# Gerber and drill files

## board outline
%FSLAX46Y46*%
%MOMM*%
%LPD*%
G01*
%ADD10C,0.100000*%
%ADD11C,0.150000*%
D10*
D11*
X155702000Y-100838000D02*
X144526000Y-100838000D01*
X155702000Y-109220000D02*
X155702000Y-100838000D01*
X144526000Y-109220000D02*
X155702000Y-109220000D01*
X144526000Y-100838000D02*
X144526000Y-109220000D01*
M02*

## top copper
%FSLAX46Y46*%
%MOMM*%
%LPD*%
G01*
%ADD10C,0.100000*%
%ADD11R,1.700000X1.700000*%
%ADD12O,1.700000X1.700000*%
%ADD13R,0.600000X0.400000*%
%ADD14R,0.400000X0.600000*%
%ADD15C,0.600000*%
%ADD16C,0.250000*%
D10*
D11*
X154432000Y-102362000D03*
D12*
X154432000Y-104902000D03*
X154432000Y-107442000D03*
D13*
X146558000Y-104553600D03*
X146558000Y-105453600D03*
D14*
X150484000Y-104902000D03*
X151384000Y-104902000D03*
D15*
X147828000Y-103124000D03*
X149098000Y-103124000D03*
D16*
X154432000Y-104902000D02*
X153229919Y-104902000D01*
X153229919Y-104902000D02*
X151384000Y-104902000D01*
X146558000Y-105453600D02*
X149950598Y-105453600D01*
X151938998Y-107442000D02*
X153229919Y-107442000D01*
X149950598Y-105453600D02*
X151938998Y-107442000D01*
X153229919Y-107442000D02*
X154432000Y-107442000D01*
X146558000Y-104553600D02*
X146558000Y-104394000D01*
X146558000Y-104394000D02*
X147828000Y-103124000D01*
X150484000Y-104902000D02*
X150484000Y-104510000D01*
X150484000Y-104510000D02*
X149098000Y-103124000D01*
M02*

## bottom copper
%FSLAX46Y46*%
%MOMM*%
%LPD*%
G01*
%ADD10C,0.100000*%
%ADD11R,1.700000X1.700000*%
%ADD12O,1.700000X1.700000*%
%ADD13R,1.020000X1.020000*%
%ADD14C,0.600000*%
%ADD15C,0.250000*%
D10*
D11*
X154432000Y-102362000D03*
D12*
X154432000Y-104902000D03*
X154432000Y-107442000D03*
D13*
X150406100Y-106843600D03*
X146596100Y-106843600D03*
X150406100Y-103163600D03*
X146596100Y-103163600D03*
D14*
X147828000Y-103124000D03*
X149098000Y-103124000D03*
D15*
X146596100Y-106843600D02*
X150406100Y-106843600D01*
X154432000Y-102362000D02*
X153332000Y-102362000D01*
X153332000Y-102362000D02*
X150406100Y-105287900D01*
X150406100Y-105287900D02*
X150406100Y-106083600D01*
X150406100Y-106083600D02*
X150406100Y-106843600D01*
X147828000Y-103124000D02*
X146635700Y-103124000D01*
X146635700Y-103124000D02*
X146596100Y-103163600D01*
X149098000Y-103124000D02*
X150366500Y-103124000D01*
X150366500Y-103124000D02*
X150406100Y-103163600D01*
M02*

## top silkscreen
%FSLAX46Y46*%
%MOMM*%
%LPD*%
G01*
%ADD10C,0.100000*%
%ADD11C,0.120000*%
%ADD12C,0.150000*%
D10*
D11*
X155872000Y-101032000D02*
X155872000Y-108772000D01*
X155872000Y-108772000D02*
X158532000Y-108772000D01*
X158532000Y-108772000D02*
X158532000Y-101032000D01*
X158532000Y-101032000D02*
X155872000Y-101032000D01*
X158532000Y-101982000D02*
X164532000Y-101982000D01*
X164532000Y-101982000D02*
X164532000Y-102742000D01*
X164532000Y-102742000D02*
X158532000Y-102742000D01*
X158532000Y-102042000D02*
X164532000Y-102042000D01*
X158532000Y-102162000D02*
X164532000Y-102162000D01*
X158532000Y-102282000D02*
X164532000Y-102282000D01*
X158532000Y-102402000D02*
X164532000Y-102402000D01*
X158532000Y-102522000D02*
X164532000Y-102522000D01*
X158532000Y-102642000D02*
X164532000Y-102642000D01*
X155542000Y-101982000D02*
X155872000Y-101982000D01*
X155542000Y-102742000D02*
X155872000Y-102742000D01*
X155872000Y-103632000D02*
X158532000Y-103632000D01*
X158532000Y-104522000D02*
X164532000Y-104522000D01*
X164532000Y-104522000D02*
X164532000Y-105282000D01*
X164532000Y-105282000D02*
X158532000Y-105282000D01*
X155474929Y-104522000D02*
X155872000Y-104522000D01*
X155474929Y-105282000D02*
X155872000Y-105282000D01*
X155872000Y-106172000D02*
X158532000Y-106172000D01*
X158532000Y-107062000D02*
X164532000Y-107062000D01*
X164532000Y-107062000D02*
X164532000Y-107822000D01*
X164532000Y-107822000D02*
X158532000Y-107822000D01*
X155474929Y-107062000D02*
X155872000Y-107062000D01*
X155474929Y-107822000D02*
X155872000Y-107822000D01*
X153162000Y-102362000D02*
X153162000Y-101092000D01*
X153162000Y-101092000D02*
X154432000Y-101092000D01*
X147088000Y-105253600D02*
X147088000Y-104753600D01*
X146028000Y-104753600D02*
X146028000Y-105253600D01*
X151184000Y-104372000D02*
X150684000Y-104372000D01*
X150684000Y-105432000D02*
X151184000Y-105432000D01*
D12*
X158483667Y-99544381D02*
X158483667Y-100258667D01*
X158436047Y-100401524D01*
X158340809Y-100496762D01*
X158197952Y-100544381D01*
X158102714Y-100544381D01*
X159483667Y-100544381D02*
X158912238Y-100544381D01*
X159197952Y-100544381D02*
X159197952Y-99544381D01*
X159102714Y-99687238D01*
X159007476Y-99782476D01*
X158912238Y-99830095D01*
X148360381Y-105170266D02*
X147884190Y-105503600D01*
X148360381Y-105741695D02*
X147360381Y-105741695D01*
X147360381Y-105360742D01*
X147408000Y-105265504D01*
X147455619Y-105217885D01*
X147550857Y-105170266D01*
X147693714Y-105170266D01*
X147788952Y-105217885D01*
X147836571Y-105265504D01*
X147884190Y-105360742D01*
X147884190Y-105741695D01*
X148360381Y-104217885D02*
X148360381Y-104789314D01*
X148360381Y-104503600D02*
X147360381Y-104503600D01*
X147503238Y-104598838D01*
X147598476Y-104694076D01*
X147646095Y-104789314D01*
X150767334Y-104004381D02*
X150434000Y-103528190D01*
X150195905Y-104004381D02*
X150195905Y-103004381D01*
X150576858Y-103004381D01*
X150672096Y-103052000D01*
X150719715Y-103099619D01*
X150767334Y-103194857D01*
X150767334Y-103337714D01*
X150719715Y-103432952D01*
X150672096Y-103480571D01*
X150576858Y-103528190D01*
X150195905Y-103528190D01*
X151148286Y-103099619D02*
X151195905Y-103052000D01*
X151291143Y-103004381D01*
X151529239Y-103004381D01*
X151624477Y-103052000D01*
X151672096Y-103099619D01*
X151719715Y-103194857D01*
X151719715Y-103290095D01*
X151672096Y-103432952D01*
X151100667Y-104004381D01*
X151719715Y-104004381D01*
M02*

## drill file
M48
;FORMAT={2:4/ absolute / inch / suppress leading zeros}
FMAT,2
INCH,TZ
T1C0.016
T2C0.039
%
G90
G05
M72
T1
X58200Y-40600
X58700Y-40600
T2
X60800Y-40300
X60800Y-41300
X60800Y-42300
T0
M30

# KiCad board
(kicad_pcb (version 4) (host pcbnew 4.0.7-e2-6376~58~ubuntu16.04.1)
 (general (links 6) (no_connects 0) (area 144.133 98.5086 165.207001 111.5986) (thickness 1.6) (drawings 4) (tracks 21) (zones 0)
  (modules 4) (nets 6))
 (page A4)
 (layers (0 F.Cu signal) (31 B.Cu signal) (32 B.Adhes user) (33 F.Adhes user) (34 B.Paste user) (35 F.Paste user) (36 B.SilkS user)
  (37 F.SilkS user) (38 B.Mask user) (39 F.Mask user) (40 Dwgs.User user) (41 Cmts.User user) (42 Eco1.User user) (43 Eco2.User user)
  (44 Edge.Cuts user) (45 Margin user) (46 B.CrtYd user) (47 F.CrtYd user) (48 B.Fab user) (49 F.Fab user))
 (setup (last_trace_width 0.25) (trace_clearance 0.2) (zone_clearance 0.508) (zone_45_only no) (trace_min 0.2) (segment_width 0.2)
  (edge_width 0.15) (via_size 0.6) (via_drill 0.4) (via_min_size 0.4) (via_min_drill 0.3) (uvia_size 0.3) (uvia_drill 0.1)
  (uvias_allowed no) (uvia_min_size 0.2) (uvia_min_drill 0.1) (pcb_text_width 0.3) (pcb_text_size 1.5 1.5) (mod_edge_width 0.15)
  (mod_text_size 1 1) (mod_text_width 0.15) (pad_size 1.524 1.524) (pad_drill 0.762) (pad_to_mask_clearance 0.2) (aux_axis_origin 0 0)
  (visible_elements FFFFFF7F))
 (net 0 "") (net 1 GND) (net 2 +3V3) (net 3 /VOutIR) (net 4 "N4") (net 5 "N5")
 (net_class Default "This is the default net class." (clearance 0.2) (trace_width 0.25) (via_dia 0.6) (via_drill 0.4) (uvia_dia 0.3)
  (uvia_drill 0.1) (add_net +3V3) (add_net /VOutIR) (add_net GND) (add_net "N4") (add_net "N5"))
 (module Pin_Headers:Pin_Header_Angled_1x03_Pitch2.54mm (layer F.Cu) (at 154.432 102.362)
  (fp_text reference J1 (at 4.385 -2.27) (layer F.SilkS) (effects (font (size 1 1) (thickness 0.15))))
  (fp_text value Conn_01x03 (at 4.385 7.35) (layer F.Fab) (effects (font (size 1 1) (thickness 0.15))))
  (fp_line (start 1.44 -1.33) (end 1.44 6.41) (layer F.SilkS) (width 0.12))
  (fp_line (start 1.44 6.41) (end 4.1 6.41) (layer F.SilkS) (width 0.12))
  (fp_line (start 4.1 6.41) (end 4.1 -1.33) (layer F.SilkS) (width 0.12))
  (fp_line (start 4.1 -1.33) (end 1.44 -1.33) (layer F.SilkS) (width 0.12))
  (fp_line (start 4.1 -0.38) (end 10.1 -0.38) (layer F.SilkS) (width 0.12))
  (fp_line (start 10.1 -0.38) (end 10.1 0.38) (layer F.SilkS) (width 0.12))
  (fp_line (start 10.1 0.38) (end 4.1 0.38) (layer F.SilkS) (width 0.12))
  (fp_line (start 4.1 -0.32) (end 10.1 -0.32) (layer F.SilkS) (width 0.12))
  (fp_line (start 4.1 -0.2) (end 10.1 -0.2) (layer F.SilkS) (width 0.12))
  (fp_line (start 4.1 -0.08) (end 10.1 -0.08) (layer F.SilkS) (width 0.12))
  (fp_line (start 4.1 0.04) (end 10.1 0.04) (layer F.SilkS) (width 0.12))
  (fp_line (start 4.1 0.16) (end 10.1 0.16) (layer F.SilkS) (width 0.12))
  (fp_line (start 4.1 0.28) (end 10.1 0.28) (layer F.SilkS) (width 0.12))
  (fp_line (start 1.11 -0.38) (end 1.44 -0.38) (layer F.SilkS) (width 0.12))
  (fp_line (start 1.11 0.38) (end 1.44 0.38) (layer F.SilkS) (width 0.12))
  (fp_line (start 1.44 1.27) (end 4.1 1.27) (layer F.SilkS) (width 0.12))
  (fp_line (start 4.1 2.16) (end 10.1 2.16) (layer F.SilkS) (width 0.12))
  (fp_line (start 10.1 2.16) (end 10.1 2.92) (layer F.SilkS) (width 0.12))
  (fp_line (start 10.1 2.92) (end 4.1 2.92) (layer F.SilkS) (width 0.12))
  (fp_line (start 1.042929 2.16) (end 1.44 2.16) (layer F.SilkS) (width 0.12))
  (fp_line (start 1.042929 2.92) (end 1.44 2.92) (layer F.SilkS) (width 0.12))
  (fp_line (start 1.44 3.81) (end 4.1 3.81) (layer F.SilkS) (width 0.12))
  (fp_line (start 4.1 4.7) (end 10.1 4.7) (layer F.SilkS) (width 0.12))
  (fp_line (start 10.1 4.7) (end 10.1 5.46) (layer F.SilkS) (width 0.12))
  (fp_line (start 10.1 5.46) (end 4.1 5.46) (layer F.SilkS) (width 0.12))
  (fp_line (start 1.042929 4.7) (end 1.44 4.7) (layer F.SilkS) (width 0.12))
  (fp_line (start 1.042929 5.46) (end 1.44 5.46) (layer F.SilkS) (width 0.12))
  (fp_line (start -1.27 0) (end -1.27 -1.27) (layer F.SilkS) (width 0.12))
  (fp_line (start -1.27 -1.27) (end 0 -1.27) (layer F.SilkS) (width 0.12))
  (pad 1 thru_hole rect (at 0 0) (size 1.7 1.7) (drill 1) (layers *.Cu *.Mask) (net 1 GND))
  (pad 2 thru_hole oval (at 0 2.54) (size 1.7 1.7) (drill 1) (layers *.Cu *.Mask) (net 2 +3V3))
  (pad 3 thru_hole oval (at 0 5.08) (size 1.7 1.7) (drill 1) (layers *.Cu *.Mask) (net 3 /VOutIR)))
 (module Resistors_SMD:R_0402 (layer F.Cu) (at 146.558 105.0036 270)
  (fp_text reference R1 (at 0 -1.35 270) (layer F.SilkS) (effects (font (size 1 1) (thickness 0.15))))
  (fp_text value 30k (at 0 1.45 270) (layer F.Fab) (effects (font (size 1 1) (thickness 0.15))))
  (fp_line (start 0.25 -0.53) (end -0.25 -0.53) (layer F.SilkS) (width 0.12))
  (fp_line (start -0.25 0.53) (end 0.25 0.53) (layer F.SilkS) (width 0.12))
  (pad 1 smd rect (at -0.45 0 270) (size 0.4 0.6) (layers F.Cu F.Paste F.Mask) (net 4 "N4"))
  (pad 2 smd rect (at 0.45 0 270) (size 0.4 0.6) (layers F.Cu F.Paste F.Mask) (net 3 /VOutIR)))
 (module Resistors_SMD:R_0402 (layer F.Cu) (at 150.934 104.902)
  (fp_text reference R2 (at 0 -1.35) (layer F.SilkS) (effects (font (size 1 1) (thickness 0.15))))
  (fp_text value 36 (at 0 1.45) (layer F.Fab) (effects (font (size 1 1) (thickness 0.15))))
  (fp_line (start 0.25 -0.53) (end -0.25 -0.53) (layer F.SilkS) (width 0.12))
  (fp_line (start -0.25 0.53) (end 0.25 0.53) (layer F.SilkS) (width 0.12))
  (pad 1 smd rect (at -0.45 0) (size 0.4 0.6) (layers F.Cu F.Paste F.Mask) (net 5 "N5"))
  (pad 2 smd rect (at 0.45 0) (size 0.4 0.6) (layers F.Cu F.Paste F.Mask) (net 2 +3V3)))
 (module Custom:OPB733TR (layer B.Cu) (at 148.5011 105.0036)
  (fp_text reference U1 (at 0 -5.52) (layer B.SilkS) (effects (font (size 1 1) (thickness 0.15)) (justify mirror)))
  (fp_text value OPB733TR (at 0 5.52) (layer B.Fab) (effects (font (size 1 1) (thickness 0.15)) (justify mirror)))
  (pad 3 smd rect (at 1.905 1.84) (size 1.02 1.02) (layers B.Cu B.Paste B.Mask) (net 1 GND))
  (pad 4 smd rect (at -1.905 1.84) (size 1.02 1.02) (layers B.Cu B.Paste B.Mask) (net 1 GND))
  (pad 2 smd rect (at 1.905 -1.84) (size 1.02 1.02) (layers B.Cu B.Paste B.Mask) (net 5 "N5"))
  (pad 1 smd rect (at -1.905 -1.84) (size 1.02 1.02) (layers B.Cu B.Paste B.Mask) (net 4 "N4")))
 (gr_line (start 155.702 100.838) (end 144.526 100.838) (layer Edge.Cuts) (width 0.15))
 (gr_line (start 155.702 109.22) (end 155.702 100.838) (layer Edge.Cuts) (width 0.15))
 (gr_line (start 144.526 109.22) (end 155.702 109.22) (layer Edge.Cuts) (width 0.15))
 (gr_line (start 144.526 100.838) (end 144.526 109.22) (layer Edge.Cuts) (width 0.15))
 (segment (start 146.5961 106.8436) (end 150.4061 106.8436) (width 0.25) (layer B.Cu) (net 1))
 (segment (start 154.432 102.362) (end 153.332 102.362) (width 0.25) (layer B.Cu) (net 1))
 (segment (start 153.332 102.362) (end 150.4061 105.2879) (width 0.25) (layer B.Cu) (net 1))
 (segment (start 150.4061 105.2879) (end 150.4061 106.0836) (width 0.25) (layer B.Cu) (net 1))
 (segment (start 150.4061 106.0836) (end 150.4061 106.8436) (width 0.25) (layer B.Cu) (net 1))
 (segment (start 154.432 104.902) (end 153.229919 104.902) (width 0.25) (layer F.Cu) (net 2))
 (segment (start 153.229919 104.902) (end 151.384 104.902) (width 0.25) (layer F.Cu) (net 2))
 (segment (start 146.558 105.4536) (end 149.950598 105.4536) (width 0.25) (layer F.Cu) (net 3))
 (segment (start 151.938998 107.442) (end 153.229919 107.442) (width 0.25) (layer F.Cu) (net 3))
 (segment (start 149.950598 105.4536) (end 151.938998 107.442) (width 0.25) (layer F.Cu) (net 3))
 (segment (start 153.229919 107.442) (end 154.432 107.442) (width 0.25) (layer F.Cu) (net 3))
 (segment (start 147.828 103.124) (end 146.6357 103.124) (width 0.25) (layer B.Cu) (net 4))
 (segment (start 146.6357 103.124) (end 146.5961 103.1636) (width 0.25) (layer B.Cu) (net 4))
 (segment (start 146.558 104.5536) (end 146.558 104.394) (width 0.25) (layer F.Cu) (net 4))
 (via (at 147.828 103.124) (size 0.6) (drill 0.4) (layers F.Cu B.Cu) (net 4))
 (segment (start 146.558 104.394) (end 147.828 103.124) (width 0.25) (layer F.Cu) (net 4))
 (segment (start 149.098 103.124) (end 150.3665 103.124) (width 0.25) (layer B.Cu) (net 5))
 (segment (start 150.3665 103.124) (end 150.4061 103.1636) (width 0.25) (layer B.Cu) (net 5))
 (segment (start 150.484 104.902) (end 150.484 104.51) (width 0.25) (layer F.Cu) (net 5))
 (segment (start 150.484 104.51) (end 149.098 103.124) (width 0.25) (layer F.Cu) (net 5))
 (via (at 149.098 103.124) (size 0.6) (drill 0.4) (layers F.Cu B.Cu) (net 5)))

